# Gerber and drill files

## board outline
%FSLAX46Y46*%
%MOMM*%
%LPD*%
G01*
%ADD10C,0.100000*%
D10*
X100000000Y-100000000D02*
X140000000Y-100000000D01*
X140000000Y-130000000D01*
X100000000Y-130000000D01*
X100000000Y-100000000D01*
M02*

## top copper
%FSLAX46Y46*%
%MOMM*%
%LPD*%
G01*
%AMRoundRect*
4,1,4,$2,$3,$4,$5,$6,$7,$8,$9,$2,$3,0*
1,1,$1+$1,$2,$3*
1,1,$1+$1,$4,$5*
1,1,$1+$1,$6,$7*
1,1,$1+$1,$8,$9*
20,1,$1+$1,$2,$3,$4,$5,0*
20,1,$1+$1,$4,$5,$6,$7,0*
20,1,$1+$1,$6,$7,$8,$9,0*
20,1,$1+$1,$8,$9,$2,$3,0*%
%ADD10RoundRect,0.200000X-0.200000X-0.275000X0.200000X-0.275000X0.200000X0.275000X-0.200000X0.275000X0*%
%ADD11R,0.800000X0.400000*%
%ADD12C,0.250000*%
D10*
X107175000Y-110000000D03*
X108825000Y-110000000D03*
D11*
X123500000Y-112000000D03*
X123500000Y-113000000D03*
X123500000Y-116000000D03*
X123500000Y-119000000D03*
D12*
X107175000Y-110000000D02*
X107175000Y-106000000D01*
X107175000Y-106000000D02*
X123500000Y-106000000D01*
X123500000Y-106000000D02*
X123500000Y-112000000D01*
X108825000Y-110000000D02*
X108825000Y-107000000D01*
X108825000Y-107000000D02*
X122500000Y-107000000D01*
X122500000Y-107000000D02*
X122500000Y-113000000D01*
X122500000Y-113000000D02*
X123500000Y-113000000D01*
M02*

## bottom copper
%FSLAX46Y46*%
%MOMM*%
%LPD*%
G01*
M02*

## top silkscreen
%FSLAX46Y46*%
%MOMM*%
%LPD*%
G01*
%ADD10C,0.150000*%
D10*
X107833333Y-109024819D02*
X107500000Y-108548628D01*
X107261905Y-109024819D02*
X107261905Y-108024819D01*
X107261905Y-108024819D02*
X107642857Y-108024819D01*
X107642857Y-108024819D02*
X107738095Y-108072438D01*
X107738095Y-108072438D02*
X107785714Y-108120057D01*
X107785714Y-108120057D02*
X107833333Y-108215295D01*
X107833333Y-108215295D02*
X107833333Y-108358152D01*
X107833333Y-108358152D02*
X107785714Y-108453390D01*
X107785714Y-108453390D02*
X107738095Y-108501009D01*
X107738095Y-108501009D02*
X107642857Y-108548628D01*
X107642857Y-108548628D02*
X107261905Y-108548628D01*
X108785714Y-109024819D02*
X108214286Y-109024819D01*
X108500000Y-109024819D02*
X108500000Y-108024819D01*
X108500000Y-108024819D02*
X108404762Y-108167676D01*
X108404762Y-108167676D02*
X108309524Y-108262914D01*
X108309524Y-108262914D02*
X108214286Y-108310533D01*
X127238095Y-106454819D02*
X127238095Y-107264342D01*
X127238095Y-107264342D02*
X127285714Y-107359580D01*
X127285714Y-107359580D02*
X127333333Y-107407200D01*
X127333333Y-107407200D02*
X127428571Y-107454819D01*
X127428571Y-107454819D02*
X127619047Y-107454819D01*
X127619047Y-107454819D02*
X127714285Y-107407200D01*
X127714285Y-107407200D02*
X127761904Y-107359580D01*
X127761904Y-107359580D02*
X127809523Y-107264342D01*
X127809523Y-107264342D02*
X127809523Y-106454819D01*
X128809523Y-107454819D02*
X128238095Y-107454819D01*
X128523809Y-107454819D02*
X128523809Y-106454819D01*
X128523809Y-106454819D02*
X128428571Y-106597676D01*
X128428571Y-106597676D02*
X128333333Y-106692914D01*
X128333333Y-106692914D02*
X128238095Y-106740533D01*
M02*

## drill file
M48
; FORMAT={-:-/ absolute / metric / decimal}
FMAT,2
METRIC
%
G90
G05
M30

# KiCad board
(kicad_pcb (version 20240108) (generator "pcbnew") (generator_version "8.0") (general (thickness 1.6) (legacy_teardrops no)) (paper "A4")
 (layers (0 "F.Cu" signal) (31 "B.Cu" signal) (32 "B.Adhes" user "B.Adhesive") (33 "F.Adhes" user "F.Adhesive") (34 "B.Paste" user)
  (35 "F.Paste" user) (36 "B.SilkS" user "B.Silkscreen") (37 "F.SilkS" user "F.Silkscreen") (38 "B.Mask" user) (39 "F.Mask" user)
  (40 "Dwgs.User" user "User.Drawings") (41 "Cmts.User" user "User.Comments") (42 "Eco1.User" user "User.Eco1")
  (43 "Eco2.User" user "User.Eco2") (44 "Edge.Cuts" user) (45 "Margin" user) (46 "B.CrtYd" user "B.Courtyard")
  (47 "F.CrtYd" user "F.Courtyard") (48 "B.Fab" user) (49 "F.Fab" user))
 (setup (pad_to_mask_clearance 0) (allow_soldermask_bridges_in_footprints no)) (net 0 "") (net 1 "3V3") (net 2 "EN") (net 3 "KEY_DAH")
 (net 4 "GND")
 (gr_rect (start 100 100) (end 140 130) (stroke (width 0.1) (type default)) (layer "Edge.Cuts"))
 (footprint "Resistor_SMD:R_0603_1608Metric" (layer "F.Cu") (at 108 110)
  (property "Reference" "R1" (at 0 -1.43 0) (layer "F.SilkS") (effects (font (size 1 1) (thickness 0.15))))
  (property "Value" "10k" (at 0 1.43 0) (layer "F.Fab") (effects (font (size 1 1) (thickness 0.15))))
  (pad "1" smd roundrect (at -0.825 0) (size 0.8 0.95) (layers "F.Cu" "F.Paste" "F.Mask") (roundrect_rratio 0.25) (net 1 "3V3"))
  (pad "2" smd roundrect (at 0.825 0) (size 0.8 0.95) (layers "F.Cu" "F.Paste" "F.Mask") (roundrect_rratio 0.25) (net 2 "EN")))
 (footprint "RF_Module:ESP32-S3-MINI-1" (layer "F.Cu") (at 128 115)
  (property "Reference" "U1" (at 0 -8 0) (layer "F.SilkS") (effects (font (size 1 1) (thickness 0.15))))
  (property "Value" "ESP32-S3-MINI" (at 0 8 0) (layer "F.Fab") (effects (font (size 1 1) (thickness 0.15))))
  (pad "1" smd rect (at -4.5 -3.0) (size 0.8 0.4) (layers "F.Cu" "F.Paste" "F.Mask") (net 1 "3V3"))
  (pad "2" smd rect (at -4.5 -2.0) (size 0.8 0.4) (layers "F.Cu" "F.Paste" "F.Mask") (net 2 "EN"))
  (pad "5" smd rect (at -4.5 1.0) (size 0.8 0.4) (layers "F.Cu" "F.Paste" "F.Mask") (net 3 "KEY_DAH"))
  (pad "8" smd rect (at -4.5 4.0) (size 0.8 0.4) (layers "F.Cu" "F.Paste" "F.Mask") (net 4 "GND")))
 (segment (start 107.175 110) (end 107.175 106) (width 0.25) (layer "F.Cu") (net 1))
 (segment (start 107.175 106) (end 123.5 106) (width 0.25) (layer "F.Cu") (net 1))
 (segment (start 123.5 106) (end 123.5 112) (width 0.25) (layer "F.Cu") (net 1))
 (segment (start 108.825 110) (end 108.825 107) (width 0.25) (layer "F.Cu") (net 2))
 (segment (start 108.825 107) (end 122.5 107) (width 0.25) (layer "F.Cu") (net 2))
 (segment (start 122.5 107) (end 122.5 113) (width 0.25) (layer "F.Cu") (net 2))
 (segment (start 122.5 113) (end 123.5 113) (width 0.25) (layer "F.Cu") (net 2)))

